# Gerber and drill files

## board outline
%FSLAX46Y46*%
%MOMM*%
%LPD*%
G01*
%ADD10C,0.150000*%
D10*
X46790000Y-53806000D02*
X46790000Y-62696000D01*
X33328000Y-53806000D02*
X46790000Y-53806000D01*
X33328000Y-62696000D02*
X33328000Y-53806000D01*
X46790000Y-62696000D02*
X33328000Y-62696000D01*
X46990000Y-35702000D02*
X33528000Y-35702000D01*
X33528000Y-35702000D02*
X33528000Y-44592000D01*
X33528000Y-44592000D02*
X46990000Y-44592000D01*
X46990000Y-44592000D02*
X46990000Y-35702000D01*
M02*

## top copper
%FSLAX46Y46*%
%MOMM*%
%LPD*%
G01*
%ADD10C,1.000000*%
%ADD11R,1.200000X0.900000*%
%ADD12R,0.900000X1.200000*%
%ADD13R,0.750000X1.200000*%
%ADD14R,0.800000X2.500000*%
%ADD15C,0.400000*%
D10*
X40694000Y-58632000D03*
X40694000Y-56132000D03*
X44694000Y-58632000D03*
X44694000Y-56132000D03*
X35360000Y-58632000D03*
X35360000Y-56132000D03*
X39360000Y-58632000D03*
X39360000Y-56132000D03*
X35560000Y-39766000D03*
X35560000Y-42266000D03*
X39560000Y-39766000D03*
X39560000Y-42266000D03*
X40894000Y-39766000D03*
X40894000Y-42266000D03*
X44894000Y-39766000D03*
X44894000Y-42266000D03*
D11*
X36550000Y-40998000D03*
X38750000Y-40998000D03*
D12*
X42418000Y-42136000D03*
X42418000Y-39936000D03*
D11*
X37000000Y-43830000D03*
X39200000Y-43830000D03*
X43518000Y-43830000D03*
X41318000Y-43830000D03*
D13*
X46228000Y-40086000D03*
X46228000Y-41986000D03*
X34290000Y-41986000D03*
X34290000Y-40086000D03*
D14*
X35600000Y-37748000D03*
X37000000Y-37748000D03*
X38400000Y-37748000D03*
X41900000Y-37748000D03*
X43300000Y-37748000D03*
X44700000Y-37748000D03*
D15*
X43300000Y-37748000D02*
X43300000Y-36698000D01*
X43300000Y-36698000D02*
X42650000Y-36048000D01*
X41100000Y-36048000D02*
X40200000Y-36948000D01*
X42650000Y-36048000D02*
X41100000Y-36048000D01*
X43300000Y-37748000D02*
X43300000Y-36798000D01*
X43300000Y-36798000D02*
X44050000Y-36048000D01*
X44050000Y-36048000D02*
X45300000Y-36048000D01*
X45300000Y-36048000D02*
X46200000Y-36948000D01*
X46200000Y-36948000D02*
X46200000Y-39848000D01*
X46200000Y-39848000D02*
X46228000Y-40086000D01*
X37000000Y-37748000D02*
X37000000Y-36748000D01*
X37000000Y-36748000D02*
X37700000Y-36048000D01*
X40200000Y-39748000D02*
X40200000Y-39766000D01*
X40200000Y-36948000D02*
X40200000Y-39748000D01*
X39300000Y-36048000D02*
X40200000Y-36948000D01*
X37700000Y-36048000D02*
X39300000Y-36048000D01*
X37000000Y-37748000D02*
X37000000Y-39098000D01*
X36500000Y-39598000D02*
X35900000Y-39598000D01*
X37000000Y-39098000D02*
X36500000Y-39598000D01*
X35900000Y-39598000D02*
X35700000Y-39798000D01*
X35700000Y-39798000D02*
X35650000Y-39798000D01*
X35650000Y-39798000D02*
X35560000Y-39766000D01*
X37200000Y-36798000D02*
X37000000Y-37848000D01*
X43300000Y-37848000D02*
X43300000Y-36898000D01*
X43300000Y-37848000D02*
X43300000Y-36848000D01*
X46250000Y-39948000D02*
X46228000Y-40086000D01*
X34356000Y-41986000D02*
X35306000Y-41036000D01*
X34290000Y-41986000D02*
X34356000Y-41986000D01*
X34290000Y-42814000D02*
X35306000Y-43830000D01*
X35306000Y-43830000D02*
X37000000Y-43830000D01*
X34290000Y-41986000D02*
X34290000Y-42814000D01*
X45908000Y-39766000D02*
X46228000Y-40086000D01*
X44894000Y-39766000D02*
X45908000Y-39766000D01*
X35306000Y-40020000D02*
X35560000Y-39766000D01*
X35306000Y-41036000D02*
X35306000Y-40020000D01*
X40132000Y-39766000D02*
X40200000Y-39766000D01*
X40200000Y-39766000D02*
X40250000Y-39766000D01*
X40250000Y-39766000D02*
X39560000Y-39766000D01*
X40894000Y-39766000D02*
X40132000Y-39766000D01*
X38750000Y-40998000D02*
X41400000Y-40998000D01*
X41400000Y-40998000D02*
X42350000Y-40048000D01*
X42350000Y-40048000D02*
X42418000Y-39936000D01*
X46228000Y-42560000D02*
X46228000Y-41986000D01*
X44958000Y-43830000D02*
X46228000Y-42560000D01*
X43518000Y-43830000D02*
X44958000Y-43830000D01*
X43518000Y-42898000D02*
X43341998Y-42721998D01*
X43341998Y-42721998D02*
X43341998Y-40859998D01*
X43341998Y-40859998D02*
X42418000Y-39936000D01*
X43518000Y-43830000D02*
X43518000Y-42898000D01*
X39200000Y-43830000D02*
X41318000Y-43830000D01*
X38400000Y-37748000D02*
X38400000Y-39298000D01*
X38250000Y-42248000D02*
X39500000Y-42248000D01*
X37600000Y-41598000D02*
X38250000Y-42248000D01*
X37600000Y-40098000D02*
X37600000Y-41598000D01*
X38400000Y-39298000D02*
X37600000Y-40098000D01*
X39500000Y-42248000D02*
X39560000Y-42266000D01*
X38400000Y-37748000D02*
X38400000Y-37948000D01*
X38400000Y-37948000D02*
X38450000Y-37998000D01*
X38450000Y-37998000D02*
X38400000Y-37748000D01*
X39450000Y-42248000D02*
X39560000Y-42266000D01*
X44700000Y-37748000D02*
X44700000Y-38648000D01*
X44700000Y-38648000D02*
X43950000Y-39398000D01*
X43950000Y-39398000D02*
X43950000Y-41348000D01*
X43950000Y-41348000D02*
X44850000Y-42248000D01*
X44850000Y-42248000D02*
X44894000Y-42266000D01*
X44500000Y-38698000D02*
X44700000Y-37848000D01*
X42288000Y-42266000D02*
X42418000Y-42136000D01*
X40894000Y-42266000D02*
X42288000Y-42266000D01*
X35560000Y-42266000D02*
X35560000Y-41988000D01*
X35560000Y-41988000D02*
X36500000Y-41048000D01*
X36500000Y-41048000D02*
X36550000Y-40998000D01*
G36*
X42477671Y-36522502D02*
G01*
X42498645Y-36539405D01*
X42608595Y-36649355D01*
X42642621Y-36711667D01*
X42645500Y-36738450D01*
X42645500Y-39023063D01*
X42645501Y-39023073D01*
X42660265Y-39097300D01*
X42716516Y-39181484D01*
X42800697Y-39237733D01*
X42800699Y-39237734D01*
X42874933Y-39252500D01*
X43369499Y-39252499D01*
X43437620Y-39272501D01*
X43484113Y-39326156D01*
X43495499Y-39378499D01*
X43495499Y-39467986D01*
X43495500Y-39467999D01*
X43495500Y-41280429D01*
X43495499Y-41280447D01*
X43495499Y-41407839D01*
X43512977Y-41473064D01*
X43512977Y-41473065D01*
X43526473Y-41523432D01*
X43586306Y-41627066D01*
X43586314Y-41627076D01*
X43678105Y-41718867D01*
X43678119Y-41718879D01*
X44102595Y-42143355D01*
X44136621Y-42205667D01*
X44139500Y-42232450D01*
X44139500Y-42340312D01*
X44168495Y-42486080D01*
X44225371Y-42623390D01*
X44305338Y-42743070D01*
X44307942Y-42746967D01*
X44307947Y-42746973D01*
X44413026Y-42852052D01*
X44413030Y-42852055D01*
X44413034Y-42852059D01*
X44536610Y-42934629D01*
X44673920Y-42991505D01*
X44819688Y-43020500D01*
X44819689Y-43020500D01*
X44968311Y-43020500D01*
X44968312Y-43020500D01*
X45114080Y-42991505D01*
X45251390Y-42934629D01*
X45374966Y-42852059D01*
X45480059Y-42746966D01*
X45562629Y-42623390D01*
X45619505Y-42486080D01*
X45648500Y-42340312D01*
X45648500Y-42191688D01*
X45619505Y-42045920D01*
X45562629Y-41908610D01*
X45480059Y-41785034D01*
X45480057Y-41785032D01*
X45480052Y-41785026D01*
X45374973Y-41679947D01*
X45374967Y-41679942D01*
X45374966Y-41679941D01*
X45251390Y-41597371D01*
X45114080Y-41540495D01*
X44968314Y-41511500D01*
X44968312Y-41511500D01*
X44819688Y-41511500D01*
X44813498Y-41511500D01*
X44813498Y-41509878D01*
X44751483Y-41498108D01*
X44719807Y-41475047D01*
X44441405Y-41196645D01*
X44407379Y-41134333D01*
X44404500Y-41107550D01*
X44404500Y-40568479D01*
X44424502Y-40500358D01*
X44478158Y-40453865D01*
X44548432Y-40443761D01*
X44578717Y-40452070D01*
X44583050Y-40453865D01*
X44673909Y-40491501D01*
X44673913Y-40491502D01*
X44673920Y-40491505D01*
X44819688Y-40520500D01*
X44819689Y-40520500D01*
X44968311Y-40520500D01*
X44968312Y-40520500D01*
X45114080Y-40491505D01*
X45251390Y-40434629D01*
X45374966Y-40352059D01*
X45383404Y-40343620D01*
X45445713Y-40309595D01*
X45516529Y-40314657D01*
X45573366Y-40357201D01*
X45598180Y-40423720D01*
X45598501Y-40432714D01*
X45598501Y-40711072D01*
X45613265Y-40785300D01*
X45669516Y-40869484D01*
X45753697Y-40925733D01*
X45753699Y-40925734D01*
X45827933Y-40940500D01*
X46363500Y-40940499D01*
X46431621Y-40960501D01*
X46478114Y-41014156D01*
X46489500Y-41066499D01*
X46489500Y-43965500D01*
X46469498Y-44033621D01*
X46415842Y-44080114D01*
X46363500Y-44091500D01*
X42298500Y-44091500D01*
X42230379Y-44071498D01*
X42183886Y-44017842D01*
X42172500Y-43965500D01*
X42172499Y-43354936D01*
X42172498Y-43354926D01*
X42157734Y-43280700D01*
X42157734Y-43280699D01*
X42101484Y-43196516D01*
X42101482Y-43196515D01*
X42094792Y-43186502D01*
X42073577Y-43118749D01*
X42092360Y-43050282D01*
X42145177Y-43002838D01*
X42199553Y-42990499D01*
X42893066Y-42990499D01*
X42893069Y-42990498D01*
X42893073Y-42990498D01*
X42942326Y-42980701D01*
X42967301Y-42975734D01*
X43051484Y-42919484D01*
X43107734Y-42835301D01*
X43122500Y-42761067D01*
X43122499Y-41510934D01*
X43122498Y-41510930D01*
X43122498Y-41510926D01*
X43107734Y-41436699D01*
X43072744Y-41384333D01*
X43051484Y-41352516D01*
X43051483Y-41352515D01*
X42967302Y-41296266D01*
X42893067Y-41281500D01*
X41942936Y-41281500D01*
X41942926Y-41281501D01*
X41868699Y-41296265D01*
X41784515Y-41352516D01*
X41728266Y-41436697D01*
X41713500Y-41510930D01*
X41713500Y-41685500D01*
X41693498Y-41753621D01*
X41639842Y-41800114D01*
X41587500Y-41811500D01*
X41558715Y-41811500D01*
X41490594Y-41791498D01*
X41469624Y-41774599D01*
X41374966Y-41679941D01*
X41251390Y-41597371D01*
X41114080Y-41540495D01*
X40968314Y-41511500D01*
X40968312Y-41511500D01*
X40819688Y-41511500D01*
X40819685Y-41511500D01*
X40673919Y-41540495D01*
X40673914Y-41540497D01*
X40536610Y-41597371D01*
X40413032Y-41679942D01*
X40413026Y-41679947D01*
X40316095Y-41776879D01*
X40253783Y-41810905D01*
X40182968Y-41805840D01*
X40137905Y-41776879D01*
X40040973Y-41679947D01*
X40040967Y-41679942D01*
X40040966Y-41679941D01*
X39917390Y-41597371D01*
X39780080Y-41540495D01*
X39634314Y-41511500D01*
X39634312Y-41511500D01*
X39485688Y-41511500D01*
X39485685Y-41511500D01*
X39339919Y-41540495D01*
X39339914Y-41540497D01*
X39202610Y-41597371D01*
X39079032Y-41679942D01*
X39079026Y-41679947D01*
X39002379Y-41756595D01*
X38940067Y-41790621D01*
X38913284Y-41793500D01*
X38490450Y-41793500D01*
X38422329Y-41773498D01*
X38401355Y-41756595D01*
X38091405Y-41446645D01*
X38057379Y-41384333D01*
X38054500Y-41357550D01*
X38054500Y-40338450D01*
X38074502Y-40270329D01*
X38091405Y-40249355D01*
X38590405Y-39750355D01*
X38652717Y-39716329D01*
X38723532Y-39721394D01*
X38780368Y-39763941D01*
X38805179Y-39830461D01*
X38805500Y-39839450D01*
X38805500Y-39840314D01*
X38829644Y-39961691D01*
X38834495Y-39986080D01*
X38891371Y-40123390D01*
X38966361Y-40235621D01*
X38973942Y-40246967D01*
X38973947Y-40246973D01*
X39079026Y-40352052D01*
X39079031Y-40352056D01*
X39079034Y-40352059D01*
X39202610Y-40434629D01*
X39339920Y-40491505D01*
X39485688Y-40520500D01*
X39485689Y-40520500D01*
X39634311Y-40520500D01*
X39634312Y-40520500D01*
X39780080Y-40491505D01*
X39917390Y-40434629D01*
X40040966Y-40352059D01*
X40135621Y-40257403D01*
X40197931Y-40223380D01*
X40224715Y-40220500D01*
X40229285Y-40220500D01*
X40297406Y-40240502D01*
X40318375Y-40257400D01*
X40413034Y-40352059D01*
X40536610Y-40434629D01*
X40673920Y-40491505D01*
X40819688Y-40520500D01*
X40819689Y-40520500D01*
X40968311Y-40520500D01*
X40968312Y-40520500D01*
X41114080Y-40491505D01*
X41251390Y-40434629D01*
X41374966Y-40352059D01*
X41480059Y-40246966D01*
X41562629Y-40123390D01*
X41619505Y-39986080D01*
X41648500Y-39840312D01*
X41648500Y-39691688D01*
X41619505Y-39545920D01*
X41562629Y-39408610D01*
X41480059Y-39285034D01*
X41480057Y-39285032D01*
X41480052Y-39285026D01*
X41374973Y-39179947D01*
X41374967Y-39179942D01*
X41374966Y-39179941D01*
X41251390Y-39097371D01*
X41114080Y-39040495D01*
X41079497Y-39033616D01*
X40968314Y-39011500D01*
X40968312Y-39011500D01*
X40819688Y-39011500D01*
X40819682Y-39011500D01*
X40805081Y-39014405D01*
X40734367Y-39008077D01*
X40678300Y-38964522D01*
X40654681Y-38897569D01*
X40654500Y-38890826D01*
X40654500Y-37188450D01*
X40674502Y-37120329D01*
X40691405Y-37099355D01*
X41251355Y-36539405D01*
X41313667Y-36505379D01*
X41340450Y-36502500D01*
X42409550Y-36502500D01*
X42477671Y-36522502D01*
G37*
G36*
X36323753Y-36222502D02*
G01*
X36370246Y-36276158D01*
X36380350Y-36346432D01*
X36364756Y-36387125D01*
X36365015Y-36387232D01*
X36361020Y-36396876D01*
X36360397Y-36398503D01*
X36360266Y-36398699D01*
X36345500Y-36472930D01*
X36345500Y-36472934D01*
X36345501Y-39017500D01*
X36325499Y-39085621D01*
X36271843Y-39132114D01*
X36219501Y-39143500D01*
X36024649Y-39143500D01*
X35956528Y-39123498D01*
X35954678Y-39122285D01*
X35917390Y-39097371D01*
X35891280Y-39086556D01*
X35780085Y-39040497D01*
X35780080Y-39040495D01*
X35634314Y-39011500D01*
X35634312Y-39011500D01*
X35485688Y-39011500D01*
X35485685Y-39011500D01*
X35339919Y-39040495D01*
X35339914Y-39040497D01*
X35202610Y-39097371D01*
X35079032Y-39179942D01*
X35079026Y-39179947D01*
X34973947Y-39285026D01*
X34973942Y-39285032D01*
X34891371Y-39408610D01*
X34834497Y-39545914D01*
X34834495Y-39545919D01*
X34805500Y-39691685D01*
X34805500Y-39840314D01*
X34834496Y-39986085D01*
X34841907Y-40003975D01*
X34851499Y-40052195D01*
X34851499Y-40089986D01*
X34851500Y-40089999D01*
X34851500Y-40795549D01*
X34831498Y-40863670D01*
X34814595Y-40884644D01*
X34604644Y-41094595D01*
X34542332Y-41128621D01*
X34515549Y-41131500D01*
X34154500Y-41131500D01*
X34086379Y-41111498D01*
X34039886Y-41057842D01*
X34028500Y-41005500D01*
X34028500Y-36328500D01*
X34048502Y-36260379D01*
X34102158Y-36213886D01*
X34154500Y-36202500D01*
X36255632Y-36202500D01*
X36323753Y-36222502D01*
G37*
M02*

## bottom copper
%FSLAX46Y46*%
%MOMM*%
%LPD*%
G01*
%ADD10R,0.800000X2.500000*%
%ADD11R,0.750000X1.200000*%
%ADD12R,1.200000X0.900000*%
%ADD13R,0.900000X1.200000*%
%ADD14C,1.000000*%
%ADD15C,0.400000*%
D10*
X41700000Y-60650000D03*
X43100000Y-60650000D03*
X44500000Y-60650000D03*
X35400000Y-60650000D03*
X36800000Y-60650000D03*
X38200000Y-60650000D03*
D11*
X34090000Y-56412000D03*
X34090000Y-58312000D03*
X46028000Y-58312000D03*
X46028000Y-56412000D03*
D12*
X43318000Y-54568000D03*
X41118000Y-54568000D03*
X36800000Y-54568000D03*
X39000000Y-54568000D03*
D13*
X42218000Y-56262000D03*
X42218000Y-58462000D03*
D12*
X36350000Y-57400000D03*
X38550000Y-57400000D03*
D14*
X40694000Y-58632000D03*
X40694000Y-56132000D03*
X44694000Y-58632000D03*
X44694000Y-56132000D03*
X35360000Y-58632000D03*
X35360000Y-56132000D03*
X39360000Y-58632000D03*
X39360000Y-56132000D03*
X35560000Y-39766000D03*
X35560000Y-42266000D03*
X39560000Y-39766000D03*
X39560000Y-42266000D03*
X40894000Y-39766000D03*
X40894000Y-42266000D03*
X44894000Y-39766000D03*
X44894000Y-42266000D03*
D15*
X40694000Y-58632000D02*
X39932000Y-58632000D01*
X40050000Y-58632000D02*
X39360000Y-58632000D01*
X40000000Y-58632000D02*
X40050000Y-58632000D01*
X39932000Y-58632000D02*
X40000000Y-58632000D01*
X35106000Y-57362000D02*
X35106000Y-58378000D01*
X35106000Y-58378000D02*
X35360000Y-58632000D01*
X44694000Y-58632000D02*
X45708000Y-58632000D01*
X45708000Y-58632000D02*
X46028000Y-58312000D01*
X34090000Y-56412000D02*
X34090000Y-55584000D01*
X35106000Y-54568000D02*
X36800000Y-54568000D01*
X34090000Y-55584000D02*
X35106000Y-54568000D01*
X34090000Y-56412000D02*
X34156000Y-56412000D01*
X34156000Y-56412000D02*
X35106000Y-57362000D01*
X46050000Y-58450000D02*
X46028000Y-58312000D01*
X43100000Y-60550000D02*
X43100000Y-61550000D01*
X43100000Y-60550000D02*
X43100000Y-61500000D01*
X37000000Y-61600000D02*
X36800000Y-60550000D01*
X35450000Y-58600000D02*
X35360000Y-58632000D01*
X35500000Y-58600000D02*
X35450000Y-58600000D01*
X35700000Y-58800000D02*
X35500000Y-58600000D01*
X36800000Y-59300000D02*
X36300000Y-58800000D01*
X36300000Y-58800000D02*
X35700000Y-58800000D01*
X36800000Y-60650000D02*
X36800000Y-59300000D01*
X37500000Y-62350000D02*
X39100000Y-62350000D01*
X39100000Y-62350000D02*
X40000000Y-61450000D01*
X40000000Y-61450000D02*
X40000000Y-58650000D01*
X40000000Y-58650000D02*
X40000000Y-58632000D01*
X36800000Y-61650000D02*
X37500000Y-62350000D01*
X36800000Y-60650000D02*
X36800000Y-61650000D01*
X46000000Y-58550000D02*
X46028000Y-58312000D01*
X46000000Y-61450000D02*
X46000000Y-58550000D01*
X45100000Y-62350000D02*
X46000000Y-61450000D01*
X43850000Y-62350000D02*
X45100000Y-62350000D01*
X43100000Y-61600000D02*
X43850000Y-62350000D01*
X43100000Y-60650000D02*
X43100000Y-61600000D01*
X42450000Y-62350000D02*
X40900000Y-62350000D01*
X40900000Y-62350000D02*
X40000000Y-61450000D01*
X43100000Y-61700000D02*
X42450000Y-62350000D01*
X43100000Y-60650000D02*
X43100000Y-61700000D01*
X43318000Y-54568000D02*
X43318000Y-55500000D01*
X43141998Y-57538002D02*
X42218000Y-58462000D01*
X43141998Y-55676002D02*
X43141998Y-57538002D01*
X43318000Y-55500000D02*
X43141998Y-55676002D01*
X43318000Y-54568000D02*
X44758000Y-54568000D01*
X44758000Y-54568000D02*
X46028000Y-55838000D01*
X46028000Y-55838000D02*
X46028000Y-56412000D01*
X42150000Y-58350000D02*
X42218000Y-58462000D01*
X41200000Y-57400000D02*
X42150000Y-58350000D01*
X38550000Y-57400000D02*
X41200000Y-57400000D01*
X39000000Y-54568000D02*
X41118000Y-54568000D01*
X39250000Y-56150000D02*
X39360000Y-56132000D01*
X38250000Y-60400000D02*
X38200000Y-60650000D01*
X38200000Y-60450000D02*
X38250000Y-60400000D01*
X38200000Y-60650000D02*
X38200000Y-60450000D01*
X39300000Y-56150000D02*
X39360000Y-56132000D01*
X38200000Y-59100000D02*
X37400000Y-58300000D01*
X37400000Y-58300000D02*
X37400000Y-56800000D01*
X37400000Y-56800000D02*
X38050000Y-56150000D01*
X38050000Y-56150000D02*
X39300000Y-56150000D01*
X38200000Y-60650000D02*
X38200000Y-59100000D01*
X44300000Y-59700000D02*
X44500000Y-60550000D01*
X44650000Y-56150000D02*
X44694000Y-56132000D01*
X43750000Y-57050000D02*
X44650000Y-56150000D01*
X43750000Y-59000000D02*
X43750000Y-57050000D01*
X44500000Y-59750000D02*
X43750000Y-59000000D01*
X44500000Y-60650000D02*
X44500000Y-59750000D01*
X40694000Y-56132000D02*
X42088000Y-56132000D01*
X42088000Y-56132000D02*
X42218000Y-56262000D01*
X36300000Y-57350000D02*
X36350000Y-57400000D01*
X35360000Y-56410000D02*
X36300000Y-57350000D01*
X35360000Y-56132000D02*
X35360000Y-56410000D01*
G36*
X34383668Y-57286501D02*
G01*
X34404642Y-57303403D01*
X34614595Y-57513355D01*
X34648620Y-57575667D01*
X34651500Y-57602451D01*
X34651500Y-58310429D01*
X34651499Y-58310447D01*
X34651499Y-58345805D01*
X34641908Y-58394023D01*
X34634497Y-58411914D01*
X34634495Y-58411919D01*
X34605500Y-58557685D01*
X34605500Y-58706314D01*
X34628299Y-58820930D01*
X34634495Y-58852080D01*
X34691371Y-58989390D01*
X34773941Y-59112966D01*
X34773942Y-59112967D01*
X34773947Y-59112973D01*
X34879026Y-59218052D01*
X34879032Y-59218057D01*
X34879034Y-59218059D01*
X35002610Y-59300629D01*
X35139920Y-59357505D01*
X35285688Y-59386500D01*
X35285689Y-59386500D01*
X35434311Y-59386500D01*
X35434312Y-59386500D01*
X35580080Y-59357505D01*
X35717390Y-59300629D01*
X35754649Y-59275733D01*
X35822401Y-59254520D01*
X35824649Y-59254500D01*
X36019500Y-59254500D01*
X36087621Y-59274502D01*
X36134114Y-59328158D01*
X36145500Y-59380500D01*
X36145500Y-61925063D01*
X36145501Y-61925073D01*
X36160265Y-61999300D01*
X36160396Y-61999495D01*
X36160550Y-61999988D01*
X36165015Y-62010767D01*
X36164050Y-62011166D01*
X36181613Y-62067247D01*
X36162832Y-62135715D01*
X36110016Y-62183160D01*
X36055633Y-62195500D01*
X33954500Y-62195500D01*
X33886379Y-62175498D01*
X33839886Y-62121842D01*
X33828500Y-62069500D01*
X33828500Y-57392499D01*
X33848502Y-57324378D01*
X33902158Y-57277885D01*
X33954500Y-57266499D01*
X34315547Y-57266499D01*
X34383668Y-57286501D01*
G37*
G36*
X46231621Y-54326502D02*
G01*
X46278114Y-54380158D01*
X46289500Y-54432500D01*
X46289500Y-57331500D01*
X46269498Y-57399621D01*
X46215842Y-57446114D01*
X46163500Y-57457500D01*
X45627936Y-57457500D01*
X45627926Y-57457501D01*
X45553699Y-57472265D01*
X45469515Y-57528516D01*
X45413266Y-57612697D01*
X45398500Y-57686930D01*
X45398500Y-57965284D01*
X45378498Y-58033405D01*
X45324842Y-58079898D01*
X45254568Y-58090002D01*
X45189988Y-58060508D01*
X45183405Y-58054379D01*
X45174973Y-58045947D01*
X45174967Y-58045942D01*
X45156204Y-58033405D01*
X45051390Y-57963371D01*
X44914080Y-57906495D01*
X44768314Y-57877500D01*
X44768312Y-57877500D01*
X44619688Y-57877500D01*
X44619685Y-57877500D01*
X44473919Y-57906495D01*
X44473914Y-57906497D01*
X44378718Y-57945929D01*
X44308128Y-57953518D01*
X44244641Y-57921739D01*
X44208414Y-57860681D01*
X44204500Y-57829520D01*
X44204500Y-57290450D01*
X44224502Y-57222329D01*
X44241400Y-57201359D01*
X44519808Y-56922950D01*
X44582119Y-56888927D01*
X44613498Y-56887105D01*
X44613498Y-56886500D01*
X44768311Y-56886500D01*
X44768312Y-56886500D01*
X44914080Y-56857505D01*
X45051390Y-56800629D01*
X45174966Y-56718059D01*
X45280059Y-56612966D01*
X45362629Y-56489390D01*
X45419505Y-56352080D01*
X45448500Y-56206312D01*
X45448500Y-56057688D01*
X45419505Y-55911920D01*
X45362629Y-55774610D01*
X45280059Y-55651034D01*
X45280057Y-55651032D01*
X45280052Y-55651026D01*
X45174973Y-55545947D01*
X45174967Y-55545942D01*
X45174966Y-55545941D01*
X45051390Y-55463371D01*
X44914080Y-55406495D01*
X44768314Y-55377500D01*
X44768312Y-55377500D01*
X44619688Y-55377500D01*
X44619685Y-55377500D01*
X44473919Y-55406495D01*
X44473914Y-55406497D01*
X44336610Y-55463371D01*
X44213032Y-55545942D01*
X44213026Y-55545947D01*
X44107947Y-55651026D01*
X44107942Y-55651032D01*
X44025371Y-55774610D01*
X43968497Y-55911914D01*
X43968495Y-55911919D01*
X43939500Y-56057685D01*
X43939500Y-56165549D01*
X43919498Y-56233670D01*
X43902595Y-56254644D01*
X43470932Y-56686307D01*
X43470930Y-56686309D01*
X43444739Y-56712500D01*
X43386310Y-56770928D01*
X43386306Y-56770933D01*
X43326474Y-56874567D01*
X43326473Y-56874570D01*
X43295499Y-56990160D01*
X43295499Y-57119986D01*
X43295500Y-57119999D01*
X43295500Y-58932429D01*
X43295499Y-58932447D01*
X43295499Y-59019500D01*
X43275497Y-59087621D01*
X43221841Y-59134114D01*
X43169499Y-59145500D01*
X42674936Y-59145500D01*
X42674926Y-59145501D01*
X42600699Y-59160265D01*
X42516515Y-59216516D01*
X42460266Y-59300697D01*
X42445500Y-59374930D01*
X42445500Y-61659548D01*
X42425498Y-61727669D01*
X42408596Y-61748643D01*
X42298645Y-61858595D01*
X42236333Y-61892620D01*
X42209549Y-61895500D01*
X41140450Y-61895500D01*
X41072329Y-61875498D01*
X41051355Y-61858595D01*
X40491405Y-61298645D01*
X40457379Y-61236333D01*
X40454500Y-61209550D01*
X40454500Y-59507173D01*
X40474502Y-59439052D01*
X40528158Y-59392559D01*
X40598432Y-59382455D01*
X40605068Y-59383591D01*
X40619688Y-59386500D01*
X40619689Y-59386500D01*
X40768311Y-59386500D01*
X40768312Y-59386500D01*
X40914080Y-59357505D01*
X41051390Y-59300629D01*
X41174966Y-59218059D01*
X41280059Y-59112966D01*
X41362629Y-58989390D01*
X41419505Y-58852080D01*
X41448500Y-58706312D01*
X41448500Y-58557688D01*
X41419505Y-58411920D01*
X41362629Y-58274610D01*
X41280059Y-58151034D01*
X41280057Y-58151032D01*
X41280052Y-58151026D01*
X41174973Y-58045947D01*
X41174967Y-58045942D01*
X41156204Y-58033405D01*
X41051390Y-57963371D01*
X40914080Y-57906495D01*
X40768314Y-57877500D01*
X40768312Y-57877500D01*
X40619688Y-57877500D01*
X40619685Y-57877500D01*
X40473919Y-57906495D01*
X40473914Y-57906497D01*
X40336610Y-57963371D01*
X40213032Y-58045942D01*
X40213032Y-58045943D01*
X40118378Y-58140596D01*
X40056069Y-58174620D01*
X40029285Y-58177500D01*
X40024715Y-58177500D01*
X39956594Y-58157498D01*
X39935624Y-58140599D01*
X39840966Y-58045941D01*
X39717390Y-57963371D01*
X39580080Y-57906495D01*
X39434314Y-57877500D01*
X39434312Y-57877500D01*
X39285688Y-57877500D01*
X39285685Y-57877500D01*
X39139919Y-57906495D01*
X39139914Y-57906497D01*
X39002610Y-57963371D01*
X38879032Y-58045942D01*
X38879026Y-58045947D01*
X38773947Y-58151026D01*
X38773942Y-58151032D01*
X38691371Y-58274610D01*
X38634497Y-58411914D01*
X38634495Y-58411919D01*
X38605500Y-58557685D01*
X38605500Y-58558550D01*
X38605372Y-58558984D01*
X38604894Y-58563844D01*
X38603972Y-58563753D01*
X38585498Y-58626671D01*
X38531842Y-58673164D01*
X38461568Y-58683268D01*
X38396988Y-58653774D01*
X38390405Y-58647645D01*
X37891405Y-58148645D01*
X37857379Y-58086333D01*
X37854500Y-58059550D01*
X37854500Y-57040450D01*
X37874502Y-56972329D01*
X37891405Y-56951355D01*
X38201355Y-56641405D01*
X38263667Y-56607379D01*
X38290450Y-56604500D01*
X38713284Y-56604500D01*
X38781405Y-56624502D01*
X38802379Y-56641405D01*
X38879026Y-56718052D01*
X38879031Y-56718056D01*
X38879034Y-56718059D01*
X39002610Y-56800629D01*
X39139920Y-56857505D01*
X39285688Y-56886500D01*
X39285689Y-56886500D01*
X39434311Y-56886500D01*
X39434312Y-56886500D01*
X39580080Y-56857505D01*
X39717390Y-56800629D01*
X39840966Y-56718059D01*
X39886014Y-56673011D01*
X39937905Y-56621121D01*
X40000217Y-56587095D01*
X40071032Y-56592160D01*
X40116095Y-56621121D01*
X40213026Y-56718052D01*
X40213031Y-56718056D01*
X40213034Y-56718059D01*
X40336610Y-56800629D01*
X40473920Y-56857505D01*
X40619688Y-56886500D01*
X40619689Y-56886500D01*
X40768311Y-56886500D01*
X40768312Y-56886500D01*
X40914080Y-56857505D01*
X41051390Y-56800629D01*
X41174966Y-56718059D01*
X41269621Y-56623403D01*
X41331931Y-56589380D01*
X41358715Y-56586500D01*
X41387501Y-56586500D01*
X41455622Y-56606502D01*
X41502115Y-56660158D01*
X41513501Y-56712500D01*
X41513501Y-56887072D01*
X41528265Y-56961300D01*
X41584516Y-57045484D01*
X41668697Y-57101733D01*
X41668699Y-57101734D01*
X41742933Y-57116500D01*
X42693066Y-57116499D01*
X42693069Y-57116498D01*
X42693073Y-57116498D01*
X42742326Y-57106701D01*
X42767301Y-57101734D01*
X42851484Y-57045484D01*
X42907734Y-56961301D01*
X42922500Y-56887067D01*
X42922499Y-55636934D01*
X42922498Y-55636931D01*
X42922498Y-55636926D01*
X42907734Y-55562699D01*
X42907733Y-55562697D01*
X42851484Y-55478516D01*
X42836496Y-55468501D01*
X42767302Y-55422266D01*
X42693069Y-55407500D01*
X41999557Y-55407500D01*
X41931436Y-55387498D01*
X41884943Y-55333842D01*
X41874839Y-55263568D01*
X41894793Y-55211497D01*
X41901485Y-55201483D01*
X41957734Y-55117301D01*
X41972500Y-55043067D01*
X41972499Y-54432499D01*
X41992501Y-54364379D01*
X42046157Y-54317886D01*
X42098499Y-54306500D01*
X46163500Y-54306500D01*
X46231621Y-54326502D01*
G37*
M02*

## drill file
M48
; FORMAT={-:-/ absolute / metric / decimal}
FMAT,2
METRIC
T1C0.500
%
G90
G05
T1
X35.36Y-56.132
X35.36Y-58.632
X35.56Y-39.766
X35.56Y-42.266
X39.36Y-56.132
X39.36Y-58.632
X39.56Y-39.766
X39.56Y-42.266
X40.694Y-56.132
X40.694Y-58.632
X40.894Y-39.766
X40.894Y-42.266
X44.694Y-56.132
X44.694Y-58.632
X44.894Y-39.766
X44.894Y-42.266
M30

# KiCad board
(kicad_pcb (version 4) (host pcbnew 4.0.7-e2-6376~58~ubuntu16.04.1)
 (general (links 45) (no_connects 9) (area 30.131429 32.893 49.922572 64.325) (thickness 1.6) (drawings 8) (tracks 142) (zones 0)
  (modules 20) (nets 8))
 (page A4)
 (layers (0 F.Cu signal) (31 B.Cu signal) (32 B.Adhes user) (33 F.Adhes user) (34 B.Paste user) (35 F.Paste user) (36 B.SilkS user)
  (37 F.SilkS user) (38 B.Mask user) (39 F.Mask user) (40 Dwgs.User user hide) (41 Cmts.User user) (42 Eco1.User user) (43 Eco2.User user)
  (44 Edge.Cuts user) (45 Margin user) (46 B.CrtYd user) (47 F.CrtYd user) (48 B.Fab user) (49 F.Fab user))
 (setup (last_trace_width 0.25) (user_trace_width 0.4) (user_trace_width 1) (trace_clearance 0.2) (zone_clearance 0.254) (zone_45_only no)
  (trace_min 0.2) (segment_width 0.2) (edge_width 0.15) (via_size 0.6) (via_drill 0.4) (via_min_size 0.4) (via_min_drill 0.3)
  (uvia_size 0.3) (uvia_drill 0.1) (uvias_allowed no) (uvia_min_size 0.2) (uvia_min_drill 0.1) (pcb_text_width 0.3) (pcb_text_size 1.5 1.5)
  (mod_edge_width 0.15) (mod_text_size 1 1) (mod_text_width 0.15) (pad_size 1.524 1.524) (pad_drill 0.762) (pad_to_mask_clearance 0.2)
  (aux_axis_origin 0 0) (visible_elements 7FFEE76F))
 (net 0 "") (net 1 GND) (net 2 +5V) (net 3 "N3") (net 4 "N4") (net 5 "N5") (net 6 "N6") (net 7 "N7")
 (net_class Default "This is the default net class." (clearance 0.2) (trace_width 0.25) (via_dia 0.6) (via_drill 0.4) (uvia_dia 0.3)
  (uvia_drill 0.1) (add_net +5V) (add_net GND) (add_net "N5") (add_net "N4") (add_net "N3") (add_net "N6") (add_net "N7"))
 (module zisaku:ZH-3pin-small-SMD (layer B.Cu) (at 46.2 58.35 180)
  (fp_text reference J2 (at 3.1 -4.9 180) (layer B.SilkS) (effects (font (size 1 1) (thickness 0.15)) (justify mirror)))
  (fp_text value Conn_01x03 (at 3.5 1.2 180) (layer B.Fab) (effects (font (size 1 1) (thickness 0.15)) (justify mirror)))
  (pad 1 smd rect (at 4.5 -2.3 180) (size 0.8 2.5) (layers B.Cu B.Paste B.Mask) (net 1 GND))
  (pad 2 smd rect (at 3.1 -2.3 180) (size 0.8 2.5) (layers B.Cu B.Paste B.Mask) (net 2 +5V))
  (pad 3 smd rect (at 1.7 -2.3 180) (size 0.8 2.5) (layers B.Cu B.Paste B.Mask) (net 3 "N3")))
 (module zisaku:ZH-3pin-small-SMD (layer B.Cu) (at 39.9 58.35 180)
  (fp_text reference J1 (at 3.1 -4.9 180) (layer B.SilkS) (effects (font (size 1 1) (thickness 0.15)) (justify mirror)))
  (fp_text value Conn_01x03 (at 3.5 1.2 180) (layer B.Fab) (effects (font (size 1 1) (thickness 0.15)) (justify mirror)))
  (pad 1 smd rect (at 4.5 -2.3 180) (size 0.8 2.5) (layers B.Cu B.Paste B.Mask) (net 1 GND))
  (pad 2 smd rect (at 3.1 -2.3 180) (size 0.8 2.5) (layers B.Cu B.Paste B.Mask) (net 2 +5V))
  (pad 3 smd rect (at 1.7 -2.3 180) (size 0.8 2.5) (layers B.Cu B.Paste B.Mask) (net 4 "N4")))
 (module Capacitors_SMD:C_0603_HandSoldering (layer B.Cu) (at 34.09 57.362 270)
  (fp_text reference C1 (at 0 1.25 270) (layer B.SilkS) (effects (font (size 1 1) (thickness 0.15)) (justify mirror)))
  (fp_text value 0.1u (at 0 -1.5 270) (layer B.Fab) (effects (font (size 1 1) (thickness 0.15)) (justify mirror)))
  (pad 1 smd rect (at -0.95 0 270) (size 1.2 0.75) (layers B.Cu B.Paste B.Mask) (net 2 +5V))
  (pad 2 smd rect (at 0.95 0 270) (size 1.2 0.75) (layers B.Cu B.Paste B.Mask) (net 1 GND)))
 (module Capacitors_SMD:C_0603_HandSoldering (layer B.Cu) (at 46.028 57.362 90)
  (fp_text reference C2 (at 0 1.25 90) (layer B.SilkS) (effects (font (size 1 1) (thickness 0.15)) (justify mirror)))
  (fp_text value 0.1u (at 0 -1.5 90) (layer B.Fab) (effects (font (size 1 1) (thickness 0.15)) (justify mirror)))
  (pad 1 smd rect (at -0.95 0 90) (size 1.2 0.75) (layers B.Cu B.Paste B.Mask) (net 2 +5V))
  (pad 2 smd rect (at 0.95 0 90) (size 1.2 0.75) (layers B.Cu B.Paste B.Mask) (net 1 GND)))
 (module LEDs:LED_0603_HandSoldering (layer B.Cu) (at 42.218 54.568 180)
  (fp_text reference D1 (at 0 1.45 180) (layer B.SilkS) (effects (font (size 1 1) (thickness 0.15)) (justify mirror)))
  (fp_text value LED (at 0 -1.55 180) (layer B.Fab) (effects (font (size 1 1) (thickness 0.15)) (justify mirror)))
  (pad 1 smd rect (at -1.1 0 180) (size 1.2 0.9) (layers B.Cu B.Paste B.Mask) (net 1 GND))
  (pad 2 smd rect (at 1.1 0 180) (size 1.2 0.9) (layers B.Cu B.Paste B.Mask) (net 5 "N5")))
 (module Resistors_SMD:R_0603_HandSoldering (layer B.Cu) (at 37.9 54.568)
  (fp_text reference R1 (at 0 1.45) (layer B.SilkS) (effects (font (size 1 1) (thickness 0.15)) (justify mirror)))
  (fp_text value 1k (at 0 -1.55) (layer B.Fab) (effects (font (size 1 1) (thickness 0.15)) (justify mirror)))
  (pad 1 smd rect (at -1.1 0) (size 1.2 0.9) (layers B.Cu B.Paste B.Mask) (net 2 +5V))
  (pad 2 smd rect (at 1.1 0) (size 1.2 0.9) (layers B.Cu B.Paste B.Mask) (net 5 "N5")))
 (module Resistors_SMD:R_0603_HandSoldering (layer B.Cu) (at 42.218 57.362 270)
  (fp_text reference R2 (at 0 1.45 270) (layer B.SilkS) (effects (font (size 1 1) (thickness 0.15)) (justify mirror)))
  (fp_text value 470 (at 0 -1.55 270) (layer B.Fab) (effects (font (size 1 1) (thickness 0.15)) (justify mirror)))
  (pad 1 smd rect (at -1.1 0 270) (size 1.2 0.9) (layers B.Cu B.Paste B.Mask) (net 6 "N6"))
  (pad 2 smd rect (at 1.1 0 270) (size 1.2 0.9) (layers B.Cu B.Paste B.Mask) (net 1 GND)))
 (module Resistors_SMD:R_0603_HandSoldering (layer B.Cu) (at 37.45 57.4)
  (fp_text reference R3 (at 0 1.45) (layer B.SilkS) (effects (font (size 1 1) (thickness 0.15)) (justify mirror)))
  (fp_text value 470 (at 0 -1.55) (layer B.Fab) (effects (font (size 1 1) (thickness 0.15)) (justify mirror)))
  (pad 1 smd rect (at -1.1 0) (size 1.2 0.9) (layers B.Cu B.Paste B.Mask) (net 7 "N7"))
  (pad 2 smd rect (at 1.1 0) (size 1.2 0.9) (layers B.Cu B.Paste B.Mask) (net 1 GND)))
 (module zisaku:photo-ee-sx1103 (layer B.Cu) (at 40.694 58.632)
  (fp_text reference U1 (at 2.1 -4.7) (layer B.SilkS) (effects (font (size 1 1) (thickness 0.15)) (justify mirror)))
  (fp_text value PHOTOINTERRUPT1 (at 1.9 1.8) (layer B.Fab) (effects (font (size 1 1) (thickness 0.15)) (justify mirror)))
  (pad 1 thru_hole circle (at 0 0) (size 1 1) (drill 0.5) (layers *.Cu *.Mask) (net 2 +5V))
  (pad 2 thru_hole circle (at 0 -2.5) (size 1 1) (drill 0.5) (layers *.Cu *.Mask) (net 6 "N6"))
  (pad 3 thru_hole circle (at 4 0) (size 1 1) (drill 0.5) (layers *.Cu *.Mask) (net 2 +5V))
  (pad 4 thru_hole circle (at 4 -2.5) (size 1 1) (drill 0.5) (layers *.Cu *.Mask) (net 3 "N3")))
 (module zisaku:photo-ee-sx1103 (layer B.Cu) (at 35.36 58.632)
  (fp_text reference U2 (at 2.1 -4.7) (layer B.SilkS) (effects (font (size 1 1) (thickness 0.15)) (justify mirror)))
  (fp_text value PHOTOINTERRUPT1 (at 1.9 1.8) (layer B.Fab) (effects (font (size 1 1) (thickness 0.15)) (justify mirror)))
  (pad 1 thru_hole circle (at 0 0) (size 1 1) (drill 0.5) (layers *.Cu *.Mask) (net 2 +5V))
  (pad 2 thru_hole circle (at 0 -2.5) (size 1 1) (drill 0.5) (layers *.Cu *.Mask) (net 7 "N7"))
  (pad 3 thru_hole circle (at 4 0) (size 1 1) (drill 0.5) (layers *.Cu *.Mask) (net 2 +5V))
  (pad 4 thru_hole circle (at 4 -2.5) (size 1 1) (drill 0.5) (layers *.Cu *.Mask) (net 4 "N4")))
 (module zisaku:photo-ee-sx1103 (layer F.Cu) (at 35.56 39.766)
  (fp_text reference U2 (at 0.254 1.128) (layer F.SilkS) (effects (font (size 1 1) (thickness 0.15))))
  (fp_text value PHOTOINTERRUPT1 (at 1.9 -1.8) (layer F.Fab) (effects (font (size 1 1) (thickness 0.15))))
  (pad 1 thru_hole circle (at 0 0) (size 1 1) (drill 0.5) (layers *.Cu *.Mask) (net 2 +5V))
  (pad 2 thru_hole circle (at 0 2.5) (size 1 1) (drill 0.5) (layers *.Cu *.Mask) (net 7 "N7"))
  (pad 3 thru_hole circle (at 4 0) (size 1 1) (drill 0.5) (layers *.Cu *.Mask) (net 2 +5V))
  (pad 4 thru_hole circle (at 4 2.5) (size 1 1) (drill 0.5) (layers *.Cu *.Mask) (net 4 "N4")))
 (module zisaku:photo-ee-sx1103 (layer F.Cu) (at 40.894 39.766)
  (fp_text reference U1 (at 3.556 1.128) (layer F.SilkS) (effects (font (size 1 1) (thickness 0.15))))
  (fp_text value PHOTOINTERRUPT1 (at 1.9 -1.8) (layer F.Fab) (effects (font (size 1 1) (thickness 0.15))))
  (pad 1 thru_hole circle (at 0 0) (size 1 1) (drill 0.5) (layers *.Cu *.Mask) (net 2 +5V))
  (pad 2 thru_hole circle (at 0 2.5) (size 1 1) (drill 0.5) (layers *.Cu *.Mask) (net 6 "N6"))
  (pad 3 thru_hole circle (at 4 0) (size 1 1) (drill 0.5) (layers *.Cu *.Mask) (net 2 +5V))
  (pad 4 thru_hole circle (at 4 2.5) (size 1 1) (drill 0.5) (layers *.Cu *.Mask) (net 3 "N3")))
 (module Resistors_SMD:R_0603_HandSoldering (layer F.Cu) (at 37.65 40.998)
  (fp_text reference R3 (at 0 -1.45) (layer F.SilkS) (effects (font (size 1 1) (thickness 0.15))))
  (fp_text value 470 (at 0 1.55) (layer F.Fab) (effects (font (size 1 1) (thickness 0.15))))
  (pad 1 smd rect (at -1.1 0) (size 1.2 0.9) (layers F.Cu F.Paste F.Mask) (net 7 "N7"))
  (pad 2 smd rect (at 1.1 0) (size 1.2 0.9) (layers F.Cu F.Paste F.Mask) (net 1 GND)))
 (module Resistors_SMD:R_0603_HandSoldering (layer F.Cu) (at 42.418 41.036 90)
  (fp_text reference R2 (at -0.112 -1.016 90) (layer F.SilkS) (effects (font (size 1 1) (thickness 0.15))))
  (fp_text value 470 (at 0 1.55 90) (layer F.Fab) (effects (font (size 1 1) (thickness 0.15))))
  (pad 1 smd rect (at -1.1 0 90) (size 1.2 0.9) (layers F.Cu F.Paste F.Mask) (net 6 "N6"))
  (pad 2 smd rect (at 1.1 0 90) (size 1.2 0.9) (layers F.Cu F.Paste F.Mask) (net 1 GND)))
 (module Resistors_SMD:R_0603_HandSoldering (layer F.Cu) (at 38.1 43.83)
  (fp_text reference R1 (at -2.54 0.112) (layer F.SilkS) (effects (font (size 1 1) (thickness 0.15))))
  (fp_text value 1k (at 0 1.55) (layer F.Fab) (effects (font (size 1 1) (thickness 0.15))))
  (pad 1 smd rect (at -1.1 0) (size 1.2 0.9) (layers F.Cu F.Paste F.Mask) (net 2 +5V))
  (pad 2 smd rect (at 1.1 0) (size 1.2 0.9) (layers F.Cu F.Paste F.Mask) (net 5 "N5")))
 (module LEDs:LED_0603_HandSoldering (layer F.Cu) (at 42.418 43.83 180)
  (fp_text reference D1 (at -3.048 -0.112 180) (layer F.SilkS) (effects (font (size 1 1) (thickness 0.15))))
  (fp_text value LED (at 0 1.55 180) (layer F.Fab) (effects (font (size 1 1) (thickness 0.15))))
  (pad 1 smd rect (at -1.1 0 180) (size 1.2 0.9) (layers F.Cu F.Paste F.Mask) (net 1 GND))
  (pad 2 smd rect (at 1.1 0 180) (size 1.2 0.9) (layers F.Cu F.Paste F.Mask) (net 5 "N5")))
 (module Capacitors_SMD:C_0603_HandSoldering (layer F.Cu) (at 46.228 41.036 270)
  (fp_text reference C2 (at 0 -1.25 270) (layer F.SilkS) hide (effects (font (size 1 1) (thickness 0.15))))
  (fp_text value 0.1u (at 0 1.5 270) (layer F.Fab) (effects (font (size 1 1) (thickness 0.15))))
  (pad 1 smd rect (at -0.95 0 270) (size 1.2 0.75) (layers F.Cu F.Paste F.Mask) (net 2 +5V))
  (pad 2 smd rect (at 0.95 0 270) (size 1.2 0.75) (layers F.Cu F.Paste F.Mask) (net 1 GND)))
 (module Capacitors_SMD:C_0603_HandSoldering (layer F.Cu) (at 34.29 41.036 90)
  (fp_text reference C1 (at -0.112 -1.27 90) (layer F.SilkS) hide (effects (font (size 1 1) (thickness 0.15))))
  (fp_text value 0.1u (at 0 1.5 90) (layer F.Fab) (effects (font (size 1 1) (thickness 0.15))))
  (pad 1 smd rect (at -0.95 0 90) (size 1.2 0.75) (layers F.Cu F.Paste F.Mask) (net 2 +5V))
  (pad 2 smd rect (at 0.95 0 90) (size 1.2 0.75) (layers F.Cu F.Paste F.Mask) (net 1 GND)))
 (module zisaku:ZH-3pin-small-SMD (layer F.Cu) (at 40.1 40.048 180)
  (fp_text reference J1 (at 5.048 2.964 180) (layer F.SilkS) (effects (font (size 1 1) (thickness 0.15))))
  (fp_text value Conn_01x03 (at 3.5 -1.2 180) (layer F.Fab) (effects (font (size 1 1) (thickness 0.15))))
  (pad 1 smd rect (at 4.5 2.3 180) (size 0.8 2.5) (layers F.Cu F.Paste F.Mask) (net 1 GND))
  (pad 2 smd rect (at 3.1 2.3 180) (size 0.8 2.5) (layers F.Cu F.Paste F.Mask) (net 2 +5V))
  (pad 3 smd rect (at 1.7 2.3 180) (size 0.8 2.5) (layers F.Cu F.Paste F.Mask) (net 4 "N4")))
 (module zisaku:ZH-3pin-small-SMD (layer F.Cu) (at 46.4 40.048 180)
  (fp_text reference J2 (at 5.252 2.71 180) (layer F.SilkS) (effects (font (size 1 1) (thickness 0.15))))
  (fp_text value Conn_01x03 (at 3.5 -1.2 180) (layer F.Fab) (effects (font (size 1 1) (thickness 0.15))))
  (pad 1 smd rect (at 4.5 2.3 180) (size 0.8 2.5) (layers F.Cu F.Paste F.Mask) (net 1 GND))
  (pad 2 smd rect (at 3.1 2.3 180) (size 0.8 2.5) (layers F.Cu F.Paste F.Mask) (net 2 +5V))
  (pad 3 smd rect (at 1.7 2.3 180) (size 0.8 2.5) (layers F.Cu F.Paste F.Mask) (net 3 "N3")))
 (gr_line (start 46.79 53.806) (end 46.79 62.696) (angle 90) (layer Edge.Cuts) (width 0.15))
 (gr_line (start 33.328 53.806) (end 46.79 53.806) (angle 90) (layer Edge.Cuts) (width 0.15))
 (gr_line (start 33.328 62.696) (end 33.328 53.806) (angle 90) (layer Edge.Cuts) (width 0.15))
 (gr_line (start 46.79 62.696) (end 33.328 62.696) (angle 90) (layer Edge.Cuts) (width 0.15))
 (gr_line (start 46.99 35.702) (end 33.528 35.702) (angle 90) (layer Edge.Cuts) (width 0.15))
 (gr_line (start 33.528 35.702) (end 33.528 44.592) (angle 90) (layer Edge.Cuts) (width 0.15))
 (gr_line (start 33.528 44.592) (end 46.99 44.592) (angle 90) (layer Edge.Cuts) (width 0.15))
 (gr_line (start 46.99 44.592) (end 46.99 35.702) (angle 90) (layer Edge.Cuts) (width 0.15))
 (segment (start 40.694 58.632) (end 39.932 58.632) (width 0.4) (layer B.Cu) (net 2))
 (segment (start 40.05 58.632) (end 39.36 58.632) (width 0.4) (layer B.Cu) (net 2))
 (segment (start 40 58.632) (end 40.05 58.632) (width 0.4) (layer B.Cu) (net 2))
 (segment (start 39.932 58.632) (end 40 58.632) (width 0.4) (layer B.Cu) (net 2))
 (segment (start 35.106 57.362) (end 35.106 58.378) (width 0.4) (layer B.Cu) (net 2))
 (segment (start 35.106 58.378) (end 35.36 58.632) (width 0.4) (layer B.Cu) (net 2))
 (segment (start 44.694 58.632) (end 45.708 58.632) (width 0.4) (layer B.Cu) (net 2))
 (segment (start 45.708 58.632) (end 46.028 58.312) (width 0.4) (layer B.Cu) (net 2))
 (segment (start 34.09 56.412) (end 34.09 55.584) (width 0.4) (layer B.Cu) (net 2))
 (segment (start 35.106 54.568) (end 36.8 54.568) (width 0.4) (layer B.Cu) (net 2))
 (segment (start 34.09 55.584) (end 35.106 54.568) (width 0.4) (layer B.Cu) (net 2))
 (segment (start 34.09 56.412) (end 34.156 56.412) (width 0.4) (layer B.Cu) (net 2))
 (segment (start 34.156 56.412) (end 35.106 57.362) (width 0.4) (layer B.Cu) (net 2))
 (segment (start 46.05 58.45) (end 46.028 58.312) (width 0.4) (layer B.Cu) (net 2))
 (segment (start 43.1 60.55) (end 43.1 61.55) (width 0.4) (layer B.Cu) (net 2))
 (segment (start 43.1 60.55) (end 43.1 61.5) (width 0.4) (layer B.Cu) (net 2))
 (segment (start 37 61.6) (end 36.8 60.55) (width 0.4) (layer B.Cu) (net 2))
 (segment (start 35.45 58.6) (end 35.36 58.632) (width 0.4) (layer B.Cu) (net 2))
 (segment (start 35.5 58.6) (end 35.45 58.6) (width 0.4) (layer B.Cu) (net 2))
 (segment (start 35.7 58.8) (end 35.5 58.6) (width 0.4) (layer B.Cu) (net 2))
 (segment (start 36.8 59.3) (end 36.3 58.8) (width 0.4) (layer B.Cu) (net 2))
 (segment (start 36.3 58.8) (end 35.7 58.8) (width 0.4) (layer B.Cu) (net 2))
 (segment (start 36.8 60.65) (end 36.8 59.3) (width 0.4) (layer B.Cu) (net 2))
 (segment (start 37.5 62.35) (end 39.1 62.35) (width 0.4) (layer B.Cu) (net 2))
 (segment (start 39.1 62.35) (end 40 61.45) (width 0.4) (layer B.Cu) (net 2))
 (segment (start 40 61.45) (end 40 58.65) (width 0.4) (layer B.Cu) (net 2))
 (segment (start 40 58.65) (end 40 58.632) (width 0.4) (layer B.Cu) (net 2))
 (segment (start 36.8 61.65) (end 37.5 62.35) (width 0.4) (layer B.Cu) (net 2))
 (segment (start 36.8 60.65) (end 36.8 61.65) (width 0.4) (layer B.Cu) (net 2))
 (segment (start 46 58.55) (end 46.028 58.312) (width 0.4) (layer B.Cu) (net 2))
 (segment (start 46 61.45) (end 46 58.55) (width 0.4) (layer B.Cu) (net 2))
 (segment (start 45.1 62.35) (end 46 61.45) (width 0.4) (layer B.Cu) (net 2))
 (segment (start 43.85 62.35) (end 45.1 62.35) (width 0.4) (layer B.Cu) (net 2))
 (segment (start 43.1 61.6) (end 43.85 62.35) (width 0.4) (layer B.Cu) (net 2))
 (segment (start 43.1 60.65) (end 43.1 61.6) (width 0.4) (layer B.Cu) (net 2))
 (segment (start 42.45 62.35) (end 40.9 62.35) (width 0.4) (layer B.Cu) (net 2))
 (segment (start 40.9 62.35) (end 40 61.45) (width 0.4) (layer B.Cu) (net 2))
 (segment (start 43.1 61.7) (end 42.45 62.35) (width 0.4) (layer B.Cu) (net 2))
 (segment (start 43.1 60.65) (end 43.1 61.7) (width 0.4) (layer B.Cu) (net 2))
 (segment (start 43.3 37.748) (end 43.3 36.698) (width 0.4) (layer F.Cu) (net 2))
 (segment (start 43.3 36.698) (end 42.65 36.048) (width 0.4) (layer F.Cu) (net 2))
 (segment (start 41.1 36.048) (end 40.2 36.948) (width 0.4) (layer F.Cu) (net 2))
 (segment (start 42.65 36.048) (end 41.1 36.048) (width 0.4) (layer F.Cu) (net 2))
 (segment (start 43.3 37.748) (end 43.3 36.798) (width 0.4) (layer F.Cu) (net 2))
 (segment (start 43.3 36.798) (end 44.05 36.048) (width 0.4) (layer F.Cu) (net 2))
 (segment (start 44.05 36.048) (end 45.3 36.048) (width 0.4) (layer F.Cu) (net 2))
 (segment (start 45.3 36.048) (end 46.2 36.948) (width 0.4) (layer F.Cu) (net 2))
 (segment (start 46.2 36.948) (end 46.2 39.848) (width 0.4) (layer F.Cu) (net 2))
 (segment (start 46.2 39.848) (end 46.228 40.086) (width 0.4) (layer F.Cu) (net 2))
 (segment (start 37 37.748) (end 37 36.748) (width 0.4) (layer F.Cu) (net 2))
 (segment (start 37 36.748) (end 37.7 36.048) (width 0.4) (layer F.Cu) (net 2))
 (segment (start 40.2 39.748) (end 40.2 39.766) (width 0.4) (layer F.Cu) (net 2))
 (segment (start 40.2 36.948) (end 40.2 39.748) (width 0.4) (layer F.Cu) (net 2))
 (segment (start 39.3 36.048) (end 40.2 36.948) (width 0.4) (layer F.Cu) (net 2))
 (segment (start 37.7 36.048) (end 39.3 36.048) (width 0.4) (layer F.Cu) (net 2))
 (segment (start 37 37.748) (end 37 39.098) (width 0.4) (layer F.Cu) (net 2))
 (segment (start 36.5 39.598) (end 35.9 39.598) (width 0.4) (layer F.Cu) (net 2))
 (segment (start 37 39.098) (end 36.5 39.598) (width 0.4) (layer F.Cu) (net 2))
 (segment (start 35.9 39.598) (end 35.7 39.798) (width 0.4) (layer F.Cu) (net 2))
 (segment (start 35.7 39.798) (end 35.65 39.798) (width 0.4) (layer F.Cu) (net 2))
 (segment (start 35.65 39.798) (end 35.56 39.766) (width 0.4) (layer F.Cu) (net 2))
 (segment (start 37.2 36.798) (end 37 37.848) (width 0.4) (layer F.Cu) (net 2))
 (segment (start 43.3 37.848) (end 43.3 36.898) (width 0.4) (layer F.Cu) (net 2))
 (segment (start 43.3 37.848) (end 43.3 36.848) (width 0.4) (layer F.Cu) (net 2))
 (segment (start 46.25 39.948) (end 46.228 40.086) (width 0.4) (layer F.Cu) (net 2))
 (segment (start 34.356 41.986) (end 35.306 41.036) (width 0.4) (layer F.Cu) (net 2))
 (segment (start 34.29 41.986) (end 34.356 41.986) (width 0.4) (layer F.Cu) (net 2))
 (segment (start 34.29 42.814) (end 35.306 43.83) (width 0.4) (layer F.Cu) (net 2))
 (segment (start 35.306 43.83) (end 37 43.83) (width 0.4) (layer F.Cu) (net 2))
 (segment (start 34.29 41.986) (end 34.29 42.814) (width 0.4) (layer F.Cu) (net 2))
 (segment (start 45.908 39.766) (end 46.228 40.086) (width 0.4) (layer F.Cu) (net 2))
 (segment (start 44.894 39.766) (end 45.908 39.766) (width 0.4) (layer F.Cu) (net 2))
 (segment (start 35.306 40.02) (end 35.56 39.766) (width 0.4) (layer F.Cu) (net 2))
 (segment (start 35.306 41.036) (end 35.306 40.02) (width 0.4) (layer F.Cu) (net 2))
 (segment (start 40.132 39.766) (end 40.2 39.766) (width 0.4) (layer F.Cu) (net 2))
 (segment (start 40.2 39.766) (end 40.25 39.766) (width 0.4) (layer F.Cu) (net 2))
 (segment (start 40.25 39.766) (end 39.56 39.766) (width 0.4) (layer F.Cu) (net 2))
 (segment (start 40.894 39.766) (end 40.132 39.766) (width 0.4) (layer F.Cu) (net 2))
 (segment (start 43.318 54.568) (end 43.318 55.5) (width 0.4) (layer B.Cu) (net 1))
 (segment (start 43.141998 57.538002) (end 42.218 58.462) (width 0.4) (layer B.Cu) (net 1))
 (segment (start 43.141998 55.676002) (end 43.141998 57.538002) (width 0.4) (layer B.Cu) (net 1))
 (segment (start 43.318 55.5) (end 43.141998 55.676002) (width 0.4) (layer B.Cu) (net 1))
 (segment (start 43.318 54.568) (end 44.758 54.568) (width 0.4) (layer B.Cu) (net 1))
 (segment (start 44.758 54.568) (end 46.028 55.838) (width 0.4) (layer B.Cu) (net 1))
 (segment (start 46.028 55.838) (end 46.028 56.412) (width 0.4) (layer B.Cu) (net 1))
 (segment (start 42.15 58.35) (end 42.218 58.462) (width 0.4) (layer B.Cu) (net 1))
 (segment (start 41.2 57.4) (end 42.15 58.35) (width 0.4) (layer B.Cu) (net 1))
 (segment (start 38.55 57.4) (end 41.2 57.4) (width 0.4) (layer B.Cu) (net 1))
 (segment (start 38.75 40.998) (end 41.4 40.998) (width 0.4) (layer F.Cu) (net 1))
 (segment (start 41.4 40.998) (end 42.35 40.048) (width 0.4) (layer F.Cu) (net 1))
 (segment (start 42.35 40.048) (end 42.418 39.936) (width 0.4) (layer F.Cu) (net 1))
 (segment (start 46.228 42.56) (end 46.228 41.986) (width 0.4) (layer F.Cu) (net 1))
 (segment (start 44.958 43.83) (end 46.228 42.56) (width 0.4) (layer F.Cu) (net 1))
 (segment (start 43.518 43.83) (end 44.958 43.83) (width 0.4) (layer F.Cu) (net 1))
 (segment (start 43.518 42.898) (end 43.341998 42.721998) (width 0.4) (layer F.Cu) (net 1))
 (segment (start 43.341998 42.721998) (end 43.341998 40.859998) (width 0.4) (layer F.Cu) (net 1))
 (segment (start 43.341998 40.859998) (end 42.418 39.936) (width 0.4) (layer F.Cu) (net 1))
 (segment (start 43.518 43.83) (end 43.518 42.898) (width 0.4) (layer F.Cu) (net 1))
 (segment (start 39 54.568) (end 41.118 54.568) (width 0.4) (layer B.Cu) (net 5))
 (segment (start 39.2 43.83) (end 41.318 43.83) (width 0.4) (layer F.Cu) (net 5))
 (segment (start 39.25 56.15) (end 39.36 56.132) (width 0.4) (layer B.Cu) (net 4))
 (segment (start 38.25 60.4) (end 38.2 60.65) (width 0.4) (layer B.Cu) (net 4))
 (segment (start 38.2 60.45) (end 38.25 60.4) (width 0.4) (layer B.Cu) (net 4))
 (segment (start 38.2 60.65) (end 38.2 60.45) (width 0.4) (layer B.Cu) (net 4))
 (segment (start 39.3 56.15) (end 39.36 56.132) (width 0.4) (layer B.Cu) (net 4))
 (segment (start 38.2 59.1) (end 37.4 58.3) (width 0.4) (layer B.Cu) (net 4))
 (segment (start 37.4 58.3) (end 37.4 56.8) (width 0.4) (layer B.Cu) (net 4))
 (segment (start 37.4 56.8) (end 38.05 56.15) (width 0.4) (layer B.Cu) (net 4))
 (segment (start 38.05 56.15) (end 39.3 56.15) (width 0.4) (layer B.Cu) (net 4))
 (segment (start 38.2 60.65) (end 38.2 59.1) (width 0.4) (layer B.Cu) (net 4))
 (segment (start 38.4 37.748) (end 38.4 39.298) (width 0.4) (layer F.Cu) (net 4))
 (segment (start 38.25 42.248) (end 39.5 42.248) (width 0.4) (layer F.Cu) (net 4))
 (segment (start 37.6 41.598) (end 38.25 42.248) (width 0.4) (layer F.Cu) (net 4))
 (segment (start 37.6 40.098) (end 37.6 41.598) (width 0.4) (layer F.Cu) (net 4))
 (segment (start 38.4 39.298) (end 37.6 40.098) (width 0.4) (layer F.Cu) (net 4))
 (segment (start 39.5 42.248) (end 39.56 42.266) (width 0.4) (layer F.Cu) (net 4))
 (segment (start 38.4 37.748) (end 38.4 37.948) (width 0.4) (layer F.Cu) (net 4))
 (segment (start 38.4 37.948) (end 38.45 37.998) (width 0.4) (layer F.Cu) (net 4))
 (segment (start 38.45 37.998) (end 38.4 37.748) (width 0.4) (layer F.Cu) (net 4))
 (segment (start 39.45 42.248) (end 39.56 42.266) (width 0.4) (layer F.Cu) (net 4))
 (segment (start 44.3 59.7) (end 44.5 60.55) (width 0.4) (layer B.Cu) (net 3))
 (segment (start 44.65 56.15) (end 44.694 56.132) (width 0.4) (layer B.Cu) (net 3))
 (segment (start 43.75 57.05) (end 44.65 56.15) (width 0.4) (layer B.Cu) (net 3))
 (segment (start 43.75 59) (end 43.75 57.05) (width 0.4) (layer B.Cu) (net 3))
 (segment (start 44.5 59.75) (end 43.75 59) (width 0.4) (layer B.Cu) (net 3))
 (segment (start 44.5 60.65) (end 44.5 59.75) (width 0.4) (layer B.Cu) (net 3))
 (segment (start 44.7 37.748) (end 44.7 38.648) (width 0.4) (layer F.Cu) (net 3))
 (segment (start 44.7 38.648) (end 43.95 39.398) (width 0.4) (layer F.Cu) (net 3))
 (segment (start 43.95 39.398) (end 43.95 41.348) (width 0.4) (layer F.Cu) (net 3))
 (segment (start 43.95 41.348) (end 44.85 42.248) (width 0.4) (layer F.Cu) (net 3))
 (segment (start 44.85 42.248) (end 44.894 42.266) (width 0.4) (layer F.Cu) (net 3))
 (segment (start 44.5 38.698) (end 44.7 37.848) (width 0.4) (layer F.Cu) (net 3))
 (segment (start 40.694 56.132) (end 42.088 56.132) (width 0.4) (layer B.Cu) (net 6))
 (segment (start 42.088 56.132) (end 42.218 56.262) (width 0.4) (layer B.Cu) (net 6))
 (segment (start 42.288 42.266) (end 42.418 42.136) (width 0.4) (layer F.Cu) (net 6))
 (segment (start 40.894 42.266) (end 42.288 42.266) (width 0.4) (layer F.Cu) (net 6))
 (segment (start 36.3 57.35) (end 36.35 57.4) (width 0.4) (layer B.Cu) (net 7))
 (segment (start 35.36 56.41) (end 36.3 57.35) (width 0.4) (layer B.Cu) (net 7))
 (segment (start 35.36 56.132) (end 35.36 56.41) (width 0.4) (layer B.Cu) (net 7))
 (segment (start 35.56 42.266) (end 35.56 41.988) (width 0.4) (layer F.Cu) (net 7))
 (segment (start 35.56 41.988) (end 36.5 41.048) (width 0.4) (layer F.Cu) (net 7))
 (segment (start 36.5 41.048) (end 36.55 40.998) (width 0.4) (layer F.Cu) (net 7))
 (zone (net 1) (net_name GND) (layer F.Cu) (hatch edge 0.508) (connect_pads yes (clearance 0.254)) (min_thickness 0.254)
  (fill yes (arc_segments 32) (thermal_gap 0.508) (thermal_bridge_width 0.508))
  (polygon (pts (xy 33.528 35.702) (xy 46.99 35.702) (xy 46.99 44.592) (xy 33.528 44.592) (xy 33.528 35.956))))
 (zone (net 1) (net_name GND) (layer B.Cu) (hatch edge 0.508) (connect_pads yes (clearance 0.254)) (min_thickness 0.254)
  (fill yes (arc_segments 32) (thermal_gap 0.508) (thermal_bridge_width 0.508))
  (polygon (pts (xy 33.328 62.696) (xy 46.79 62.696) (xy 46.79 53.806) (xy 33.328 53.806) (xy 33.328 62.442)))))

